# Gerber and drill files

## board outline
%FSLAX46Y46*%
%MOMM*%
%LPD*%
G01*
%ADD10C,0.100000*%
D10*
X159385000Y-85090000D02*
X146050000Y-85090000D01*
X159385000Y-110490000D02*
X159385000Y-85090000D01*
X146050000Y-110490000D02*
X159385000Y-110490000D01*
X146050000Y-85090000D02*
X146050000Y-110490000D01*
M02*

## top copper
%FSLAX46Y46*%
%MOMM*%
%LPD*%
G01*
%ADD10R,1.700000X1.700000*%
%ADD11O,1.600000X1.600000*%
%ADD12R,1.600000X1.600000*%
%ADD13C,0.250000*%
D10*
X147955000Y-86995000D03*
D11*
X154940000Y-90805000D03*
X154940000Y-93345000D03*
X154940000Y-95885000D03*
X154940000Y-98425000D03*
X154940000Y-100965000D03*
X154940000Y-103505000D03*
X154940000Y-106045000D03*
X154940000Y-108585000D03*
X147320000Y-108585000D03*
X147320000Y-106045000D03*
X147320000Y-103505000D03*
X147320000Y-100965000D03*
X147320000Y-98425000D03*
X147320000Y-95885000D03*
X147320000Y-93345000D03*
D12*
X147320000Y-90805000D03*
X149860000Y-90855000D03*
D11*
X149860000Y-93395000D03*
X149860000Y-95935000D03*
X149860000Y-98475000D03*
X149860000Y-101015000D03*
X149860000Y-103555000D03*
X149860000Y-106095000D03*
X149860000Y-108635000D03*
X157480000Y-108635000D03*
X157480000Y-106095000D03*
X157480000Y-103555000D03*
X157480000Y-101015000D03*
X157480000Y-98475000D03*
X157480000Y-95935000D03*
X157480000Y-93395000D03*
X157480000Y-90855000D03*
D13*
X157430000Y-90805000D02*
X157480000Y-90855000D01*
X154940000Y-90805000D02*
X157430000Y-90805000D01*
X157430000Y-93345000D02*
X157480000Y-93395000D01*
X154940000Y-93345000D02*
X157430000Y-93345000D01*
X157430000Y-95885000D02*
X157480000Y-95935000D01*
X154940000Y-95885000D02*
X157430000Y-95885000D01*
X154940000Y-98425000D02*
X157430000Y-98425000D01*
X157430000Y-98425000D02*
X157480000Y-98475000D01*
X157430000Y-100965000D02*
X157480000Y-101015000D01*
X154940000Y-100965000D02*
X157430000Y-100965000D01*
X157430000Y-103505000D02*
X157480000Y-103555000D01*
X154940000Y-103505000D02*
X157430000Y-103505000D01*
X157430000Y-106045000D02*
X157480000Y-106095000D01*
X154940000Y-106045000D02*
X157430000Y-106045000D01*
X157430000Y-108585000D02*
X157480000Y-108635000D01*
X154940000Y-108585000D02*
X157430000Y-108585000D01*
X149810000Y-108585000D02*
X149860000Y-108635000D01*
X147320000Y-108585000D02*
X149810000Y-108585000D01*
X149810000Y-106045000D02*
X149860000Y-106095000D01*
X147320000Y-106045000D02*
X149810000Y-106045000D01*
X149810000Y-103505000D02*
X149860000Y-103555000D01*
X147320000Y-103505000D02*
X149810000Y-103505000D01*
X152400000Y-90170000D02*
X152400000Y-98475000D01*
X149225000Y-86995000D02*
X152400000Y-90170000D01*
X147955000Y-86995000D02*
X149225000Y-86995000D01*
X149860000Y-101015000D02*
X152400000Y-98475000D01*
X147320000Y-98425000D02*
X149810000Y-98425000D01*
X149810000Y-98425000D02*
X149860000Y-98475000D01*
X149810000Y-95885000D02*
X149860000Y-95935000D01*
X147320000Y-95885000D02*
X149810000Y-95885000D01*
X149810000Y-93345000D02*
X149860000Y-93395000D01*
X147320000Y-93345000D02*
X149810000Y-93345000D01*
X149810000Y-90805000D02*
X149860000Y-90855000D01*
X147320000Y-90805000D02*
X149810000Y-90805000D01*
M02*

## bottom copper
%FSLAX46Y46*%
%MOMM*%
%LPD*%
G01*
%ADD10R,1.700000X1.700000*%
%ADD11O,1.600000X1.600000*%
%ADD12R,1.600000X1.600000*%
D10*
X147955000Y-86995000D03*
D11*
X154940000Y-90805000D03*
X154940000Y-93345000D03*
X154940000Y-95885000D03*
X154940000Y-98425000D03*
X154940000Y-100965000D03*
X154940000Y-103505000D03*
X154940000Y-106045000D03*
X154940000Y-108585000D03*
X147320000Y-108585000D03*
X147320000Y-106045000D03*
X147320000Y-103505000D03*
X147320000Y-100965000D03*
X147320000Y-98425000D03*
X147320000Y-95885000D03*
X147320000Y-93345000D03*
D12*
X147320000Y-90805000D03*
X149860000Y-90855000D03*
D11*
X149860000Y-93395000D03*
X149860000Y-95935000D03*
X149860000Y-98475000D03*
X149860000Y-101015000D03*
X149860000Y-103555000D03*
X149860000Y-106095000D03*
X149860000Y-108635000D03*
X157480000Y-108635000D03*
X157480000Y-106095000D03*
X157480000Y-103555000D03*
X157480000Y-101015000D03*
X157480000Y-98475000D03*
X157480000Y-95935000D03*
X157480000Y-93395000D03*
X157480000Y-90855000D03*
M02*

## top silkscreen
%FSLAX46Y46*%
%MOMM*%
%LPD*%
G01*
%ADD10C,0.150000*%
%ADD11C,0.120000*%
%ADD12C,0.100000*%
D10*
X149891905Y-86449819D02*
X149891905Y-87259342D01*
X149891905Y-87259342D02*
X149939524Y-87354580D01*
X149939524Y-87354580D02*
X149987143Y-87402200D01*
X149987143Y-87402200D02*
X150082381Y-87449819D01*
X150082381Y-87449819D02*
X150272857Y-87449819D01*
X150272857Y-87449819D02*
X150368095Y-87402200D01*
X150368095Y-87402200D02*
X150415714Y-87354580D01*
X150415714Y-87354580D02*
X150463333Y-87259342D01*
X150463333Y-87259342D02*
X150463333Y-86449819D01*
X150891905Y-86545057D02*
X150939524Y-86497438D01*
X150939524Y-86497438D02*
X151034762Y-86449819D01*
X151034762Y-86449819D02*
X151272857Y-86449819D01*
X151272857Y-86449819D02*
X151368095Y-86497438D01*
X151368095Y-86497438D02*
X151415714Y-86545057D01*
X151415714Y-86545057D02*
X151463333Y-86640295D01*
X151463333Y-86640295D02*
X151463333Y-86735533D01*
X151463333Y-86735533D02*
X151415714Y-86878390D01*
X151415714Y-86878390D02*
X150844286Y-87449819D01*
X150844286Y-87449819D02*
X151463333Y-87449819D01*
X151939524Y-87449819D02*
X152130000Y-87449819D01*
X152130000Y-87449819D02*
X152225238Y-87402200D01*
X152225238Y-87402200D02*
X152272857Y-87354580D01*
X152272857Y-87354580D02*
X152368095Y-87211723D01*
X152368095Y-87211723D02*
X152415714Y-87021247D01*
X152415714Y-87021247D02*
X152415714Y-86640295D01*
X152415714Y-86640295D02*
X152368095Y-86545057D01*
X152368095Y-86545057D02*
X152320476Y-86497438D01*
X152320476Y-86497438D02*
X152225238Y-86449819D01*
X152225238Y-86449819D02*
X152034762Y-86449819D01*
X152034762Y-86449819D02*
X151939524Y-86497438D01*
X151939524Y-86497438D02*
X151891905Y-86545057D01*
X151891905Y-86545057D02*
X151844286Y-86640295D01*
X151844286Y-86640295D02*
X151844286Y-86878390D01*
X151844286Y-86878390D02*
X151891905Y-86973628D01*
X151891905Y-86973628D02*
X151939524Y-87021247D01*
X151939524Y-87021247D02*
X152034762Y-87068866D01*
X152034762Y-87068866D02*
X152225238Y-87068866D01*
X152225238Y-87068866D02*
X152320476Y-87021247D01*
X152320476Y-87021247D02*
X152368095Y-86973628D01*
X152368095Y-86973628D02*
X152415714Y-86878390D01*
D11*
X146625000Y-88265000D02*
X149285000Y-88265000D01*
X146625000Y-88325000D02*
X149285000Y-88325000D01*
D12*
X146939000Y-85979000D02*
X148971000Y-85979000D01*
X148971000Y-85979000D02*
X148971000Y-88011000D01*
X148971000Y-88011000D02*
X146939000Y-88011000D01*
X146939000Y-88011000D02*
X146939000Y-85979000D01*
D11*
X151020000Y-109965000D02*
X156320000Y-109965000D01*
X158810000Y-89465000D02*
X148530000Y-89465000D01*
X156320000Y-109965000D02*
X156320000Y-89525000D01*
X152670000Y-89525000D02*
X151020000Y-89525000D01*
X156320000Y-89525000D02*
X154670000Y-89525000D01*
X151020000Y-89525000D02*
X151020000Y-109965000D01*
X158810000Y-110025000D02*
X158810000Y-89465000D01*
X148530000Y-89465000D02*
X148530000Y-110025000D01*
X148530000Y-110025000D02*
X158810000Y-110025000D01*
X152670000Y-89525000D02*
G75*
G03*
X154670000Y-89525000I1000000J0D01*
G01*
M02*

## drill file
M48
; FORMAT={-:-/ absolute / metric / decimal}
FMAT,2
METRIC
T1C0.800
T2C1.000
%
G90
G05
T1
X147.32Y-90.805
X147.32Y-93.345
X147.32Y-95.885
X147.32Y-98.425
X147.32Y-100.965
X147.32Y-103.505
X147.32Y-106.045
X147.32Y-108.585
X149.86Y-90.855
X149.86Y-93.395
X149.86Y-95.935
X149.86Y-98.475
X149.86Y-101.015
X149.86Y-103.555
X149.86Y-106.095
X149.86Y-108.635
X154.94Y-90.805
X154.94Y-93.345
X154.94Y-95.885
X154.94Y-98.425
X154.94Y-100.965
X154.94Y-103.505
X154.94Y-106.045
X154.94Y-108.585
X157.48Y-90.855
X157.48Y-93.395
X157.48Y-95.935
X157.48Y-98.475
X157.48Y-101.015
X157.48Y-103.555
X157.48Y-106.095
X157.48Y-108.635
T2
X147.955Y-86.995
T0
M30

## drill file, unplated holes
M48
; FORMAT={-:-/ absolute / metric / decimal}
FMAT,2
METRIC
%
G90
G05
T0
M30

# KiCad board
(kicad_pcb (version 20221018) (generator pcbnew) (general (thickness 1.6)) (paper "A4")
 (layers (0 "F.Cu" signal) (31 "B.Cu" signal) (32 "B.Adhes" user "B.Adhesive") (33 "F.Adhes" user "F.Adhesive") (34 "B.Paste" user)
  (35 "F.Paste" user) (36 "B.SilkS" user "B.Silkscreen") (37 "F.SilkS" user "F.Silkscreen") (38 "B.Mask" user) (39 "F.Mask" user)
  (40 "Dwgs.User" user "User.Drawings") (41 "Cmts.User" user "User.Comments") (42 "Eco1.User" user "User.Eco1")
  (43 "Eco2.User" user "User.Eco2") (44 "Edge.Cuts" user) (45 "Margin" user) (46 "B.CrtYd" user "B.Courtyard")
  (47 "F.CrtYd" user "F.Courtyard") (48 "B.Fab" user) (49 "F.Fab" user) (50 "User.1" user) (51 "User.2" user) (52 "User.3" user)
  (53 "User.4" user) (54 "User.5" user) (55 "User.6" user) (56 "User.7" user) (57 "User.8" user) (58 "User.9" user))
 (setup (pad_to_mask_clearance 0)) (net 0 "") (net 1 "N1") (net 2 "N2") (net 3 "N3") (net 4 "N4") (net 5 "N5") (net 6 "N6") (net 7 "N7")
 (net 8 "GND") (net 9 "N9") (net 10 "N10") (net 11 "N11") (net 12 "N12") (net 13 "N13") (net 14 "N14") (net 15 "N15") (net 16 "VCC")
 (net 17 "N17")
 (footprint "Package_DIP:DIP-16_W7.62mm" (layer "F.Cu") (at 147.32 90.805)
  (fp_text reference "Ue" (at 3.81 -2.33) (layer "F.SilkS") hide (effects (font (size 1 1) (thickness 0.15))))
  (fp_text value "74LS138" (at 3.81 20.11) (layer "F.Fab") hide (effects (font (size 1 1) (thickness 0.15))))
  (pad "1" thru_hole rect (at 0 0) (size 1.6 1.6) (drill 0.8) (layers "*.Cu" "*.Mask") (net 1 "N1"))
  (pad "2" thru_hole oval (at 0 2.54) (size 1.6 1.6) (drill 0.8) (layers "*.Cu" "*.Mask") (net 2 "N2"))
  (pad "3" thru_hole oval (at 0 5.08) (size 1.6 1.6) (drill 0.8) (layers "*.Cu" "*.Mask") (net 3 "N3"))
  (pad "4" thru_hole oval (at 0 7.62) (size 1.6 1.6) (drill 0.8) (layers "*.Cu" "*.Mask") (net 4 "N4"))
  (pad "5" thru_hole oval (at 0 10.16) (size 1.6 1.6) (drill 0.8) (layers "*.Cu" "*.Mask") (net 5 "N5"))
  (pad "6" thru_hole oval (at 0 12.7) (size 1.6 1.6) (drill 0.8) (layers "*.Cu" "*.Mask") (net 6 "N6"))
  (pad "7" thru_hole oval (at 0 15.24) (size 1.6 1.6) (drill 0.8) (layers "*.Cu" "*.Mask") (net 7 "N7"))
  (pad "8" thru_hole oval (at 0 17.78) (size 1.6 1.6) (drill 0.8) (layers "*.Cu" "*.Mask") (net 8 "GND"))
  (pad "9" thru_hole oval (at 7.62 17.78) (size 1.6 1.6) (drill 0.8) (layers "*.Cu" "*.Mask") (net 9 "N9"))
  (pad "10" thru_hole oval (at 7.62 15.24) (size 1.6 1.6) (drill 0.8) (layers "*.Cu" "*.Mask") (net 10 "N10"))
  (pad "11" thru_hole oval (at 7.62 12.7) (size 1.6 1.6) (drill 0.8) (layers "*.Cu" "*.Mask") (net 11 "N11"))
  (pad "12" thru_hole oval (at 7.62 10.16) (size 1.6 1.6) (drill 0.8) (layers "*.Cu" "*.Mask") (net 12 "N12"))
  (pad "13" thru_hole oval (at 7.62 7.62) (size 1.6 1.6) (drill 0.8) (layers "*.Cu" "*.Mask") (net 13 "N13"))
  (pad "14" thru_hole oval (at 7.62 5.08) (size 1.6 1.6) (drill 0.8) (layers "*.Cu" "*.Mask") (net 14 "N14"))
  (pad "15" thru_hole oval (at 7.62 2.54) (size 1.6 1.6) (drill 0.8) (layers "*.Cu" "*.Mask") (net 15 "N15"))
  (pad "16" thru_hole oval (at 7.62 0) (size 1.6 1.6) (drill 0.8) (layers "*.Cu" "*.Mask") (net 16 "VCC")))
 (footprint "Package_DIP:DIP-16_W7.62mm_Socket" (layer "F.Cu") (at 149.86 90.855)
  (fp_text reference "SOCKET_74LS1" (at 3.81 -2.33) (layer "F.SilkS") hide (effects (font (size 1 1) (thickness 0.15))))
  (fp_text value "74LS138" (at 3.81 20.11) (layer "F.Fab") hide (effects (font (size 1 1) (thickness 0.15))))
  (fp_line (start -1.33 -1.39) (end -1.33 19.17) (stroke (width 0.12) (type solid)) (layer "F.SilkS"))
  (fp_line (start -1.33 19.17) (end 8.95 19.17) (stroke (width 0.12) (type solid)) (layer "F.SilkS"))
  (fp_line (start 1.16 -1.33) (end 1.16 19.11) (stroke (width 0.12) (type solid)) (layer "F.SilkS"))
  (fp_line (start 1.16 19.11) (end 6.46 19.11) (stroke (width 0.12) (type solid)) (layer "F.SilkS"))
  (fp_line (start 2.81 -1.33) (end 1.16 -1.33) (stroke (width 0.12) (type solid)) (layer "F.SilkS"))
  (fp_line (start 6.46 -1.33) (end 4.81 -1.33) (stroke (width 0.12) (type solid)) (layer "F.SilkS"))
  (fp_line (start 6.46 19.11) (end 6.46 -1.33) (stroke (width 0.12) (type solid)) (layer "F.SilkS"))
  (fp_line (start 8.95 -1.39) (end -1.33 -1.39) (stroke (width 0.12) (type solid)) (layer "F.SilkS"))
  (fp_line (start 8.95 19.17) (end 8.95 -1.39) (stroke (width 0.12) (type solid)) (layer "F.SilkS"))
  (fp_arc (start 4.81 -1.33) (mid 3.81 -0.33) (end 2.81 -1.33) (stroke (width 0.12) (type solid)) (layer "F.SilkS"))
  (pad "1" thru_hole rect (at 0 0) (size 1.6 1.6) (drill 0.8) (layers "*.Cu" "*.Mask") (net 1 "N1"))
  (pad "2" thru_hole oval (at 0 2.54) (size 1.6 1.6) (drill 0.8) (layers "*.Cu" "*.Mask") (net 2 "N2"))
  (pad "3" thru_hole oval (at 0 5.08) (size 1.6 1.6) (drill 0.8) (layers "*.Cu" "*.Mask") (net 3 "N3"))
  (pad "4" thru_hole oval (at 0 7.62) (size 1.6 1.6) (drill 0.8) (layers "*.Cu" "*.Mask") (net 4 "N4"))
  (pad "5" thru_hole oval (at 0 10.16) (size 1.6 1.6) (drill 0.8) (layers "*.Cu" "*.Mask") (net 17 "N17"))
  (pad "6" thru_hole oval (at 0 12.7) (size 1.6 1.6) (drill 0.8) (layers "*.Cu" "*.Mask") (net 6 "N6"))
  (pad "7" thru_hole oval (at 0 15.24) (size 1.6 1.6) (drill 0.8) (layers "*.Cu" "*.Mask") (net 7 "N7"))
  (pad "8" thru_hole oval (at 0 17.78) (size 1.6 1.6) (drill 0.8) (layers "*.Cu" "*.Mask") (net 8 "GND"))
  (pad "9" thru_hole oval (at 7.62 17.78) (size 1.6 1.6) (drill 0.8) (layers "*.Cu" "*.Mask") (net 9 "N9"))
  (pad "10" thru_hole oval (at 7.62 15.24) (size 1.6 1.6) (drill 0.8) (layers "*.Cu" "*.Mask") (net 10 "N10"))
  (pad "11" thru_hole oval (at 7.62 12.7) (size 1.6 1.6) (drill 0.8) (layers "*.Cu" "*.Mask") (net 11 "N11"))
  (pad "12" thru_hole oval (at 7.62 10.16) (size 1.6 1.6) (drill 0.8) (layers "*.Cu" "*.Mask") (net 12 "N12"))
  (pad "13" thru_hole oval (at 7.62 7.62) (size 1.6 1.6) (drill 0.8) (layers "*.Cu" "*.Mask") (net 13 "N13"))
  (pad "14" thru_hole oval (at 7.62 5.08) (size 1.6 1.6) (drill 0.8) (layers "*.Cu" "*.Mask") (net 14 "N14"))
  (pad "15" thru_hole oval (at 7.62 2.54) (size 1.6 1.6) (drill 0.8) (layers "*.Cu" "*.Mask") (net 15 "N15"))
  (pad "16" thru_hole oval (at 7.62 0) (size 1.6 1.6) (drill 0.8) (layers "*.Cu" "*.Mask") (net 16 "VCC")))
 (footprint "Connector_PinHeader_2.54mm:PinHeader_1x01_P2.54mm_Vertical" (layer "F.Cu") (at 147.955 86.995)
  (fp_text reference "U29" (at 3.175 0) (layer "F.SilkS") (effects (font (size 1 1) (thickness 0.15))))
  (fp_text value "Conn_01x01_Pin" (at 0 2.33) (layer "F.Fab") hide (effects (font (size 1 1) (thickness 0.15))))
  (fp_line (start -1.33 1.27) (end 1.33 1.27) (stroke (width 0.12) (type solid)) (layer "F.SilkS"))
  (fp_line (start -1.33 1.33) (end 1.33 1.33) (stroke (width 0.12) (type solid)) (layer "F.SilkS"))
  (fp_rect (start -1.016 -1.016) (end 1.016 1.016) (stroke (width 0.1) (type default)) (fill none) (layer "F.SilkS"))
  (pad "1" thru_hole rect (at 0 0) (size 1.7 1.7) (drill 1) (layers "*.Cu" "*.Mask") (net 17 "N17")))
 (gr_line (start 146.05 110.49) (end 159.385 110.49) (stroke (width 0.1) (type default)) (layer "Edge.Cuts"))
 (gr_line (start 159.385 85.09) (end 146.05 85.09) (stroke (width 0.1) (type default)) (layer "Edge.Cuts"))
 (gr_line (start 159.385 110.49) (end 159.385 85.09) (stroke (width 0.1) (type default)) (layer "Edge.Cuts"))
 (gr_line (start 146.05 85.09) (end 146.05 110.49) (stroke (width 0.1) (type default)) (layer "Edge.Cuts"))
 (segment (start 149.86 101.015) (end 152.4 98.475) (width 0.25) (layer "F.Cu") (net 17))
 (segment (start 152.4 90.17) (end 152.4 98.475) (width 0.25) (layer "F.Cu") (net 17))
 (segment (start 149.225 86.995) (end 152.4 90.17) (width 0.25) (layer "F.Cu") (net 17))
 (segment (start 147.955 86.995) (end 149.225 86.995) (width 0.25) (layer "F.Cu") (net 17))
 (segment (start 149.81 90.805) (end 149.86 90.855) (width 0.25) (layer "F.Cu") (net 1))
 (segment (start 147.32 90.805) (end 149.81 90.805) (width 0.25) (layer "F.Cu") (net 1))
 (segment (start 149.81 93.345) (end 149.86 93.395) (width 0.25) (layer "F.Cu") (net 2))
 (segment (start 147.32 93.345) (end 149.81 93.345) (width 0.25) (layer "F.Cu") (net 2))
 (segment (start 147.32 95.885) (end 149.81 95.885) (width 0.25) (layer "F.Cu") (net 3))
 (segment (start 149.81 95.885) (end 149.86 95.935) (width 0.25) (layer "F.Cu") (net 3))
 (segment (start 147.32 98.425) (end 149.81 98.425) (width 0.25) (layer "F.Cu") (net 4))
 (segment (start 149.81 98.425) (end 149.86 98.475) (width 0.25) (layer "F.Cu") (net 4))
 (segment (start 149.81 103.505) (end 149.86 103.555) (width 0.25) (layer "F.Cu") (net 6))
 (segment (start 147.32 103.505) (end 149.81 103.505) (width 0.25) (layer "F.Cu") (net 6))
 (segment (start 147.32 106.045) (end 149.81 106.045) (width 0.25) (layer "F.Cu") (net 7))
 (segment (start 149.81 106.045) (end 149.86 106.095) (width 0.25) (layer "F.Cu") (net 7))
 (segment (start 149.81 108.585) (end 149.86 108.635) (width 0.25) (layer "F.Cu") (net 8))
 (segment (start 147.32 108.585) (end 149.81 108.585) (width 0.25) (layer "F.Cu") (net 8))
 (segment (start 154.94 108.585) (end 157.43 108.585) (width 0.25) (layer "F.Cu") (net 9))
 (segment (start 157.43 108.585) (end 157.48 108.635) (width 0.25) (layer "F.Cu") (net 9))
 (segment (start 157.43 106.045) (end 157.48 106.095) (width 0.25) (layer "F.Cu") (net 10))
 (segment (start 154.94 106.045) (end 157.43 106.045) (width 0.25) (layer "F.Cu") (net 10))
 (segment (start 154.94 103.505) (end 157.43 103.505) (width 0.25) (layer "F.Cu") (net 11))
 (segment (start 157.43 103.505) (end 157.48 103.555) (width 0.25) (layer "F.Cu") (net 11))
 (segment (start 157.43 100.965) (end 157.48 101.015) (width 0.25) (layer "F.Cu") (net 12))
 (segment (start 154.94 100.965) (end 157.43 100.965) (width 0.25) (layer "F.Cu") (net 12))
 (segment (start 154.94 98.425) (end 157.43 98.425) (width 0.25) (layer "F.Cu") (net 13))
 (segment (start 157.43 98.425) (end 157.48 98.475) (width 0.25) (layer "F.Cu") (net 13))
 (segment (start 157.43 95.885) (end 157.48 95.935) (width 0.25) (layer "F.Cu") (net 14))
 (segment (start 154.94 95.885) (end 157.43 95.885) (width 0.25) (layer "F.Cu") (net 14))
 (segment (start 154.94 93.345) (end 157.43 93.345) (width 0.25) (layer "F.Cu") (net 15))
 (segment (start 157.43 93.345) (end 157.48 93.395) (width 0.25) (layer "F.Cu") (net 15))
 (segment (start 154.94 90.805) (end 157.43 90.805) (width 0.25) (layer "F.Cu") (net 16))
 (segment (start 157.43 90.805) (end 157.48 90.855) (width 0.25) (layer "F.Cu") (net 16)))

